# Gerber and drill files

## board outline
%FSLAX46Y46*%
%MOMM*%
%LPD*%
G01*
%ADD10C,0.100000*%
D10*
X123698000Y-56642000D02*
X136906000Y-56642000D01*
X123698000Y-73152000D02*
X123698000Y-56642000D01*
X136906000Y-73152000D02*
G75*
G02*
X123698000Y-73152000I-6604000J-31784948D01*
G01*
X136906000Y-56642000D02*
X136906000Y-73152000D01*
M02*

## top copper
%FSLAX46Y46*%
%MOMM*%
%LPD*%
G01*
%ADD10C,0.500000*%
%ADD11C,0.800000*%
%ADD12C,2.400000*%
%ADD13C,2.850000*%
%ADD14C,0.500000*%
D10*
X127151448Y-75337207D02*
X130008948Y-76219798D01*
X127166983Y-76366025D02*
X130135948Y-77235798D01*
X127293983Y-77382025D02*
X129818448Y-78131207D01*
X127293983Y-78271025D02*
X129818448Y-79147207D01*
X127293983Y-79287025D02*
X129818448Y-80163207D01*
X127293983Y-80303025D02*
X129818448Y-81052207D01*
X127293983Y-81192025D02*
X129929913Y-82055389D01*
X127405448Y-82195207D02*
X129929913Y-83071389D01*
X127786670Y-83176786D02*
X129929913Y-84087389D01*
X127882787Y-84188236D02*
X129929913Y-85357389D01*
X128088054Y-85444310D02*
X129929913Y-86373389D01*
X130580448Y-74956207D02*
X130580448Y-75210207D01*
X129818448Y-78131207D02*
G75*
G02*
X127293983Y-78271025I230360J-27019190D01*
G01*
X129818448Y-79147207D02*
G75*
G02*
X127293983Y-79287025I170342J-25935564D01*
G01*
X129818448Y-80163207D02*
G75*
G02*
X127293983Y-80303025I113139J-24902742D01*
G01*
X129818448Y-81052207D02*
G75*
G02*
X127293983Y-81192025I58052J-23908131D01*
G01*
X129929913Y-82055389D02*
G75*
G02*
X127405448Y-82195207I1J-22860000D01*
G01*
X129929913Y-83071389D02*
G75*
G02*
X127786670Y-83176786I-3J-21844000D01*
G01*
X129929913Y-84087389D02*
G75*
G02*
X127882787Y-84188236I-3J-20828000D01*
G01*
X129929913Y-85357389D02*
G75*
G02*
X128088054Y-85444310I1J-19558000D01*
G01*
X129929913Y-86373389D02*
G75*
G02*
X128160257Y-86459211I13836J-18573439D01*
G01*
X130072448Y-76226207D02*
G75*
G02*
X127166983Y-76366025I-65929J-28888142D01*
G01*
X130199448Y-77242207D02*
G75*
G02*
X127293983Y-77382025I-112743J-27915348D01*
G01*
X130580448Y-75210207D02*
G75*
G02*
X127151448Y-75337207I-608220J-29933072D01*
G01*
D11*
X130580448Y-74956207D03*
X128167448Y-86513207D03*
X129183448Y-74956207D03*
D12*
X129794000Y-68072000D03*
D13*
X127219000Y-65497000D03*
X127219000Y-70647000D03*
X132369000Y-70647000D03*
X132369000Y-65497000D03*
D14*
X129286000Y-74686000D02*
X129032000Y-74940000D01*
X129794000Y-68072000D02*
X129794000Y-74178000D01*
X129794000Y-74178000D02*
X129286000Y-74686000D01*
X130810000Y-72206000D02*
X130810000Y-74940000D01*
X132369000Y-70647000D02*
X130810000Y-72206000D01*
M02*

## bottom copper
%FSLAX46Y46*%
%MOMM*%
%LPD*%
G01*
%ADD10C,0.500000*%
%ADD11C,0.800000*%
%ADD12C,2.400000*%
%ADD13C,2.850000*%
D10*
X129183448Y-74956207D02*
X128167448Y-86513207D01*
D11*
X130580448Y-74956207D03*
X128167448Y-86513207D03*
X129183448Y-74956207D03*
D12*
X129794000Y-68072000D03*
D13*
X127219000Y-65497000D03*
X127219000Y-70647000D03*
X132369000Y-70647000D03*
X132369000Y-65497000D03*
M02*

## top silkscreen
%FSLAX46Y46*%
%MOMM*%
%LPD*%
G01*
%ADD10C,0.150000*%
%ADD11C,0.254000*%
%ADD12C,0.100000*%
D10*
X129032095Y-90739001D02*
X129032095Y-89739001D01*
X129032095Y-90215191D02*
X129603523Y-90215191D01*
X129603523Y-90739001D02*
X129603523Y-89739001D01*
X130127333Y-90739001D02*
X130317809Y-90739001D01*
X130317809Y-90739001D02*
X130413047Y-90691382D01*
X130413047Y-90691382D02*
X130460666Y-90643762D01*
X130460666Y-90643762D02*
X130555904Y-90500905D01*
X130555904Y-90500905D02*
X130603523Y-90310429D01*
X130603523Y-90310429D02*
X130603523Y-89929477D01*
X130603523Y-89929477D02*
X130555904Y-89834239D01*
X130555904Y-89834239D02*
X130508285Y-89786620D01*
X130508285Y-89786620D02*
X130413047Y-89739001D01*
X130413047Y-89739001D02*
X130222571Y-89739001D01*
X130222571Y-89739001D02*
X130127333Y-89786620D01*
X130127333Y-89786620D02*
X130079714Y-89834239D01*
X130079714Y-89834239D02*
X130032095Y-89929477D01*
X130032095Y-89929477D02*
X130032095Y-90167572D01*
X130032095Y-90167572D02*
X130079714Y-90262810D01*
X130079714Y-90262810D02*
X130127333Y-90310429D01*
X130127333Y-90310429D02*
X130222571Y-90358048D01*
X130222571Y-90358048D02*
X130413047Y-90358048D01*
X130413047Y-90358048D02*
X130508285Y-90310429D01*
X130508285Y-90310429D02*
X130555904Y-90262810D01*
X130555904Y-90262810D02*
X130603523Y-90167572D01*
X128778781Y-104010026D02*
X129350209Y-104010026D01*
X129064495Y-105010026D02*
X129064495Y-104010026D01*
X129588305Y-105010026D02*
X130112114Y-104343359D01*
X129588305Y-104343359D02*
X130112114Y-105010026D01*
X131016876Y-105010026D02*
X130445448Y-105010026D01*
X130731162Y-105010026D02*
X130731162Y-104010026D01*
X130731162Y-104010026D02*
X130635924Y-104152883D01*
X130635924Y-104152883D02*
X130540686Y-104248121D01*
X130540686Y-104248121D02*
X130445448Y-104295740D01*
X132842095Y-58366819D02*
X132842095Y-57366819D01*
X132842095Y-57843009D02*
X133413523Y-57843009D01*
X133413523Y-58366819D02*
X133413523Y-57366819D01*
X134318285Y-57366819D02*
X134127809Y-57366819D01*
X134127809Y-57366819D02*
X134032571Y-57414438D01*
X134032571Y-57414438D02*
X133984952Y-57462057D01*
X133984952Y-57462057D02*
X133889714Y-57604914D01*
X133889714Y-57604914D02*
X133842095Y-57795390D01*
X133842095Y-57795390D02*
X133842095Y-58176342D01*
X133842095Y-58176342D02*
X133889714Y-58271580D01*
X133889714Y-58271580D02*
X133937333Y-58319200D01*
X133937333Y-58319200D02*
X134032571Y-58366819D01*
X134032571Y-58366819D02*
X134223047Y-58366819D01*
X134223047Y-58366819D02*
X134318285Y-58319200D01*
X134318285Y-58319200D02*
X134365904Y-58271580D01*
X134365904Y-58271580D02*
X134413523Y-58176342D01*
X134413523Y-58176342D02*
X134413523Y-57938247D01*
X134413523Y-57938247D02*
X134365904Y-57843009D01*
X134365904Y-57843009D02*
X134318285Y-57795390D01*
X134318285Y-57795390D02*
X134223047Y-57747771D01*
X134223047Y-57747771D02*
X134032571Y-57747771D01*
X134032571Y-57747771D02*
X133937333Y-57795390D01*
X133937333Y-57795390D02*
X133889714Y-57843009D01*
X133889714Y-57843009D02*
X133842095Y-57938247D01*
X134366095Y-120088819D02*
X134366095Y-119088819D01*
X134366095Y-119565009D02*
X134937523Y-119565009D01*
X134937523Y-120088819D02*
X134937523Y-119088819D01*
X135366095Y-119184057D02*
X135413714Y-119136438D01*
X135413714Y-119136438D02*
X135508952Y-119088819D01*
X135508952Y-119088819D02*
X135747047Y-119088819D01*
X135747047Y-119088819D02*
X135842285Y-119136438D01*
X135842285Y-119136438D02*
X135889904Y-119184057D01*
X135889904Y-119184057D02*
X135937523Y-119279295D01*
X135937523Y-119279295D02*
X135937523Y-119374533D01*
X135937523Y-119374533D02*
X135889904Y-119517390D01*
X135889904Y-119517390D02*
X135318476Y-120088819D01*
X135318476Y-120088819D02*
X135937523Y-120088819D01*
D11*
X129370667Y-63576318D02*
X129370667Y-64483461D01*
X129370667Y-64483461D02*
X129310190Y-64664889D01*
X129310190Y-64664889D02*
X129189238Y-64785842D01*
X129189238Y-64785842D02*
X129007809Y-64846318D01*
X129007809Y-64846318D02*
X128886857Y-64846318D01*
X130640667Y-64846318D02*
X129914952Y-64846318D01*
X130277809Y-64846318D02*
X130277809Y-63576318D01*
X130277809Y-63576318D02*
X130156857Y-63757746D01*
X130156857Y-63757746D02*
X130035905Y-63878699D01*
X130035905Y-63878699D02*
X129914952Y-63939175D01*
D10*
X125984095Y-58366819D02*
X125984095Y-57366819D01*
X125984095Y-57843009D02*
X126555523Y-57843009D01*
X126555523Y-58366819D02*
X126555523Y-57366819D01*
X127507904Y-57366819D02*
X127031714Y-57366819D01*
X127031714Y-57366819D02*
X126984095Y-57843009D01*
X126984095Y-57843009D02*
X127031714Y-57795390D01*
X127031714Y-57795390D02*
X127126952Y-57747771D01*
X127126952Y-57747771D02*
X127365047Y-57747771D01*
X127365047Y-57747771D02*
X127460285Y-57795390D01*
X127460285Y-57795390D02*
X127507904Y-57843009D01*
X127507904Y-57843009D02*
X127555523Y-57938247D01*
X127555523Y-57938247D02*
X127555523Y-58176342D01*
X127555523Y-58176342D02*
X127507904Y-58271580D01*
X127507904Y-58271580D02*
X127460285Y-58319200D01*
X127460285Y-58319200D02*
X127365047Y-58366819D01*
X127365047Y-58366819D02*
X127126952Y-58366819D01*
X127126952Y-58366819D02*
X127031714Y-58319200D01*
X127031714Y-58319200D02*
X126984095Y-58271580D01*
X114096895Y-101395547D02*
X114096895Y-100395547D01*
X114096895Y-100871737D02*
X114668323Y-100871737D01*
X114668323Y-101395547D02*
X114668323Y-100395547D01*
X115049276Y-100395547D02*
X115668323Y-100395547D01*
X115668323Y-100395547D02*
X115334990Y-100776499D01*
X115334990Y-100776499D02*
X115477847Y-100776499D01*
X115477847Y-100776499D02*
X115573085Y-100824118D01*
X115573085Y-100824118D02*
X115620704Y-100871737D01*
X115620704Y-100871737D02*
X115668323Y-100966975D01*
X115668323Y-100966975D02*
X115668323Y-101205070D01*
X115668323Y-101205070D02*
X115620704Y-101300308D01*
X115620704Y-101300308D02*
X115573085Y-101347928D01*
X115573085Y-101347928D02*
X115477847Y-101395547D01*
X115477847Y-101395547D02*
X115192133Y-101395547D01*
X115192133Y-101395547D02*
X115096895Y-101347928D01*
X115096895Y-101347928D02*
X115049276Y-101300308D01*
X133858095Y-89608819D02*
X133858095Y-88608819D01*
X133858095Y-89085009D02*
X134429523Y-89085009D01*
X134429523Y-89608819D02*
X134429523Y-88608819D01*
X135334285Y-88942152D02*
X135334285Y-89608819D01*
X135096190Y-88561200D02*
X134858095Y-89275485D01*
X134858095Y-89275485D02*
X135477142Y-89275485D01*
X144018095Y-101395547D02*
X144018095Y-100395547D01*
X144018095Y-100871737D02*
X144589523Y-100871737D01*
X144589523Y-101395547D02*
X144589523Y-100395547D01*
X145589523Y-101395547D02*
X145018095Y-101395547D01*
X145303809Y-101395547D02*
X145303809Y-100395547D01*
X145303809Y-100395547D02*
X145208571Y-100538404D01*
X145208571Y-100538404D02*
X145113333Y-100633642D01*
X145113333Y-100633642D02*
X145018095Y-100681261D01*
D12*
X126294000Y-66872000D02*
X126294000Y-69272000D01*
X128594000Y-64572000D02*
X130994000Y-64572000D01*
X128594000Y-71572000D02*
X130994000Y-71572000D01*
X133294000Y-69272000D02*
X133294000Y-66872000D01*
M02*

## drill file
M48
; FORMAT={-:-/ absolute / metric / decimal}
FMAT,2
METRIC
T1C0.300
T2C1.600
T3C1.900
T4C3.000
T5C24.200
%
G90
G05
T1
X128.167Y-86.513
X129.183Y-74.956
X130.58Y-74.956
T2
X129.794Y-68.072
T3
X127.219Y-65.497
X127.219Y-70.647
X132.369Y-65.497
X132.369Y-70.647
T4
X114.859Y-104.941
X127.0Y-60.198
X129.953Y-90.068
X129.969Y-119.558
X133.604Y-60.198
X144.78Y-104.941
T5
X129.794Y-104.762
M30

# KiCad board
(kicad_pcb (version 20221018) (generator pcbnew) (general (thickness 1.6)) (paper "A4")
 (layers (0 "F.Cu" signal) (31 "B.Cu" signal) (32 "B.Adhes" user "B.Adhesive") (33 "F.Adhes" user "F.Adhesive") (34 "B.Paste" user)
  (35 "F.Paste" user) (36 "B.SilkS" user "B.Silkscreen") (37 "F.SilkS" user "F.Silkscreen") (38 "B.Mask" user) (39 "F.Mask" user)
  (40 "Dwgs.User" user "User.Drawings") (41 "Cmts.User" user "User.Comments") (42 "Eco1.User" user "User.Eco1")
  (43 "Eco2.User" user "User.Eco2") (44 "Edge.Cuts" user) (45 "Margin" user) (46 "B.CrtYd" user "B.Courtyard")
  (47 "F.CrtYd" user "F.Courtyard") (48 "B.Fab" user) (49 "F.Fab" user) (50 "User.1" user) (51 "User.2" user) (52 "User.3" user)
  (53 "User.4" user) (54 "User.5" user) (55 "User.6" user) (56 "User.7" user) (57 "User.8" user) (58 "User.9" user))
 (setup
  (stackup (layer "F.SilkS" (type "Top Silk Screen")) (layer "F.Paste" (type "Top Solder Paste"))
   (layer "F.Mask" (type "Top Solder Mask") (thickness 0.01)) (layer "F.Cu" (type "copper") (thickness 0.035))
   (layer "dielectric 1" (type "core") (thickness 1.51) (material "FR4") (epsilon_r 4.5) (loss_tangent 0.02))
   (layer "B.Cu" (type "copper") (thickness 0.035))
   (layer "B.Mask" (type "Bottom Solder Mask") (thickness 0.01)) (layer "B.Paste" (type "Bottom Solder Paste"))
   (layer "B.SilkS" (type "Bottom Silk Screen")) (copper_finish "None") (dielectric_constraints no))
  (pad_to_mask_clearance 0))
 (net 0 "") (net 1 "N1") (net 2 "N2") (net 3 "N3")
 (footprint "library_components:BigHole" (layer "F.Cu") (at 129.794 104.762182)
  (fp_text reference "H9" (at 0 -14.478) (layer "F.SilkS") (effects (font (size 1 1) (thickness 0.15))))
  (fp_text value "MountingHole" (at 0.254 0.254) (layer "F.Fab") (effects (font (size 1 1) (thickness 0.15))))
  (pad "" np_thru_hole circle (at 0 0) (size 6 6) (drill 24.2) (layers "F&B.Cu" "*.Mask")))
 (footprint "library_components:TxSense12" (layer "F.Cu") (at 129.945448 105.055207)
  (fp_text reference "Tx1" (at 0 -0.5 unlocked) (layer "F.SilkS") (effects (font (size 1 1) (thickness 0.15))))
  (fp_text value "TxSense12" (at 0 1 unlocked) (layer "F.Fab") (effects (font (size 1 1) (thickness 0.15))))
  (fp_line (start -2.794 -29.718) (end 0.0635 -28.835409) (stroke (width 0.5) (type solid)) (layer "F.Cu"))
  (fp_line (start -2.778465 -28.689182) (end 0.1905 -27.819409) (stroke (width 0.5) (type solid)) (layer "F.Cu"))
  (fp_line (start -2.651465 -27.673182) (end -0.127 -26.924) (stroke (width 0.5) (type solid)) (layer "F.Cu"))
  (fp_line (start -2.651465 -26.784182) (end -0.127 -25.908) (stroke (width 0.5) (type solid)) (layer "F.Cu"))
  (fp_line (start -2.651465 -25.768182) (end -0.127 -24.892) (stroke (width 0.5) (type solid)) (layer "F.Cu"))
  (fp_line (start -2.651465 -24.752182) (end -0.127 -24.003) (stroke (width 0.5) (type solid)) (layer "F.Cu"))
  (fp_line (start -2.651465 -23.863182) (end -0.015535 -22.999818) (stroke (width 0.5) (type solid)) (layer "F.Cu"))
  (fp_line (start -2.54 -22.86) (end -0.015535 -21.983818) (stroke (width 0.5) (type solid)) (layer "F.Cu"))
  (fp_line (start -2.158778 -21.878421) (end -0.015535 -20.967818) (stroke (width 0.5) (type solid)) (layer "F.Cu"))
  (fp_line (start -2.062661 -20.866971) (end -0.015535 -19.697818) (stroke (width 0.5) (type solid)) (layer "F.Cu"))
  (fp_line (start -1.857394 -19.610897) (end -0.015535 -18.681818) (stroke (width 0.5) (type solid)) (layer "F.Cu"))
  (fp_line (start 0.635 -30.099) (end 0.635 -29.845) (stroke (width 0.5) (type solid)) (layer "F.Cu"))
  (fp_arc (start -0.127 -26.924) (mid 1.597589 27.074015) (end -2.651465 -26.784182) (stroke (width 0.5) (type solid)) (layer "F.Cu"))
  (fp_arc (start -0.127 -25.908) (mid 1.477621 25.923999) (end -2.651465 -25.768182) (stroke (width 0.5) (type solid)) (layer "F.Cu"))
  (fp_arc (start -0.127 -24.892) (mid 1.363286 24.875633) (end -2.651465 -24.752182) (stroke (width 0.5) (type solid)) (layer "F.Cu"))
  (fp_arc (start -0.127 -24.003) (mid 1.253186 23.776747) (end -2.651465 -23.863182) (stroke (width 0.5) (type solid)) (layer "F.Cu"))
  (fp_arc (start -0.015535 -22.999818) (mid 1.248634 22.685201) (end -2.54 -22.86) (stroke (width 0.5) (type solid)) (layer "F.Cu"))
  (fp_arc (start -0.015535 -21.983818) (mid 1.057375 21.677817) (end -2.158778 -21.878421) (stroke (width 0.5) (type solid)) (layer "F.Cu"))
  (fp_arc (start -0.015535 -20.967818) (mid 1.009263 20.662955) (end -2.062661 -20.866971) (stroke (width 0.5) (type solid)) (layer "F.Cu"))
  (fp_arc (start -0.015535 -19.697818) (mid 0.906421 19.39644) (end -1.857394 -19.610897) (stroke (width 0.5) (type solid)) (layer "F.Cu"))
  (fp_arc (start -0.015535 -18.681818) (mid 0.897989 18.443262) (end -1.785191 -18.595996) (stroke (width 0.5) (type solid)) (layer "F.Cu"))
  (fp_arc (start 0.127 -28.829) (mid 1.449635 28.913968) (end -2.778465 -28.689182) (stroke (width 0.5) (type solid)) (layer "F.Cu"))
  (fp_arc (start 0.254 -27.813) (mid 1.483069 27.985657) (end -2.651465 -27.673182) (stroke (width 0.5) (type solid)) (layer "F.Cu"))
  (fp_arc (start 0.635 -29.845) (mid 1.134881 30.006809) (end -2.794 -29.718) (stroke (width 0.5) (type solid)) (layer "F.Cu"))
  (fp_line (start -0.762 -30.099) (end -1.778 -18.542) (stroke (width 0.5) (type solid)) (layer "B.Cu"))
  (pad "1" thru_hole circle (at 0.635 -30.099) (size 0.8 0.8) (drill 0.3) (layers "*.Cu" "*.Mask" "B.SilkS") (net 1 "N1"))
  (pad "2" thru_hole circle (at -1.778 -18.542) (size 0.8 0.8) (drill 0.3) (layers "*.Cu" "*.Mask") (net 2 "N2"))
  (pad "3" thru_hole circle (at -0.762 -30.099) (size 0.8 0.8) (drill 0.3) (layers "*.Cu" "*.Mask") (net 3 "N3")))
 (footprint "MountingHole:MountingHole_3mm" (layer "F.Cu") (at 133.604 60.198)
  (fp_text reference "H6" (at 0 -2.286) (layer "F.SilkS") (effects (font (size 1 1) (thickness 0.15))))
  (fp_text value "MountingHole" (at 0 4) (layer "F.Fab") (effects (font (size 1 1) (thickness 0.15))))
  (pad "" np_thru_hole circle (at 0 0) (size 3 3) (drill 3) (layers "*.Cu" "*.Mask")))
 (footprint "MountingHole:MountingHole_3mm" (layer "F.Cu") (at 129.968924 119.5578)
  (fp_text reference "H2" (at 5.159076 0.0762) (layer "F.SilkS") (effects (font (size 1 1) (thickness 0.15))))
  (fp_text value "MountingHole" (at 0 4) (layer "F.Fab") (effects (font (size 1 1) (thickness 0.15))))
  (pad "" np_thru_hole circle (at 0 0) (size 3 3) (drill 3) (layers "*.Cu" "*.Mask")))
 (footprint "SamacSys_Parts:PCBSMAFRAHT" (layer "F.Cu") (at 129.794 68.072)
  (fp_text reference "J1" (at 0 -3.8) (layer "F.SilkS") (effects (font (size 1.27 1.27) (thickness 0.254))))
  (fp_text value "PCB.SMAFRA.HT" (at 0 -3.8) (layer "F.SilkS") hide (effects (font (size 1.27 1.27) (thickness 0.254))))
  (fp_line (start -3.5 -1.2) (end -3.5 1.2) (stroke (width 0.1) (type solid)) (layer "F.SilkS"))
  (fp_line (start -1.2 -3.5) (end 1.2 -3.5) (stroke (width 0.1) (type solid)) (layer "F.SilkS"))
  (fp_line (start -1.2 3.5) (end 1.2 3.5) (stroke (width 0.1) (type solid)) (layer "F.SilkS"))
  (fp_line (start 3.5 1.2) (end 3.5 -1.2) (stroke (width 0.1) (type solid)) (layer "F.SilkS"))
  (pad "1" thru_hole circle (at 0 0) (size 2.4 2.4) (drill 1.6) (layers "*.Cu" "*.Mask") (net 3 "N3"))
  (pad "2" thru_hole circle (at -2.575 -2.575) (size 2.85 2.85) (drill 1.9) (layers "*.Cu" "*.Mask") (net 1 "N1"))
  (pad "3" thru_hole circle (at -2.575 2.575) (size 2.85 2.85) (drill 1.9) (layers "*.Cu" "*.Mask") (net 1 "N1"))
  (pad "4" thru_hole circle (at 2.575 2.575) (size 2.85 2.85) (drill 1.9) (layers "*.Cu" "*.Mask") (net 1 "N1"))
  (pad "5" thru_hole circle (at 2.575 -2.575) (size 2.85 2.85) (drill 1.9) (layers "*.Cu" "*.Mask") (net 1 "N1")))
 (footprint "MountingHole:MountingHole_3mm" (layer "F.Cu") (at 127 60.198)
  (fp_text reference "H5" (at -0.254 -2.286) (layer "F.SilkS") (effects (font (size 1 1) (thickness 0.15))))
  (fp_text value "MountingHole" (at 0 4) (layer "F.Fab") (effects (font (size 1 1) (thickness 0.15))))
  (pad "" np_thru_hole circle (at 0 0) (size 3 3) (drill 3) (layers "*.Cu" "*.Mask")))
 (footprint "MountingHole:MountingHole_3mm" (layer "F.Cu") (at 114.8588 104.940728)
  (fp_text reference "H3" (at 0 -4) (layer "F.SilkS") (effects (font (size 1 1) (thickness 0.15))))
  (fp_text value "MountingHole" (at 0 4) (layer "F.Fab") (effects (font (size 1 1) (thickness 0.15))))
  (pad "" np_thru_hole circle (at 0 0) (size 3 3) (drill 3) (layers "*.Cu" "*.Mask")))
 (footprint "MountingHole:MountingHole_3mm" (layer "F.Cu") (at 129.953383 90.0684)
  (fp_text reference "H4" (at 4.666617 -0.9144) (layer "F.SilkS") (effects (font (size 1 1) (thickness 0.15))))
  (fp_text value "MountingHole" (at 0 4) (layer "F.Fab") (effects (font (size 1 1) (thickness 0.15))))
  (pad "" np_thru_hole circle (at 0 0) (size 3 3) (drill 3) (layers "*.Cu" "*.Mask")))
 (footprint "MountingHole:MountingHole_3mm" (layer "F.Cu") (at 144.78 104.940728)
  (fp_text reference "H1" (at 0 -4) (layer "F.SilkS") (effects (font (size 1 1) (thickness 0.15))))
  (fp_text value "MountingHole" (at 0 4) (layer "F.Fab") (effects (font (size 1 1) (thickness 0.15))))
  (pad "" np_thru_hole circle (at 0 0) (size 3 3) (drill 3) (layers "*.Cu" "*.Mask")))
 (gr_line (start 123.698 56.642) (end 136.906 56.642) (stroke (width 0.1) (type solid)) (layer "Edge.Cuts"))
 (gr_line (start 123.698 73.152) (end 123.698 56.642) (stroke (width 0.1) (type solid)) (layer "Edge.Cuts"))
 (gr_arc (start 136.906 73.152) (mid 130.302 137.400708) (end 123.698 73.152) (stroke (width 0.1) (type solid)) (layer "Edge.Cuts"))
 (gr_line (start 136.906 56.642) (end 136.906 73.152) (stroke (width 0.1) (type solid)) (layer "Edge.Cuts"))
 (segment (start 129.286 74.686) (end 129.032 74.94) (width 0.5) (layer "F.Cu") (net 3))
 (segment (start 129.794 68.072) (end 129.794 74.178) (width 0.5) (layer "F.Cu") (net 3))
 (segment (start 129.794 74.178) (end 129.286 74.686) (width 0.5) (layer "F.Cu") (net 3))
 (segment (start 130.81 72.206) (end 130.81 74.94) (width 0.5) (layer "F.Cu") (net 1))
 (segment (start 132.369 70.647) (end 130.81 72.206) (width 0.5) (layer "F.Cu") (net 1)))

